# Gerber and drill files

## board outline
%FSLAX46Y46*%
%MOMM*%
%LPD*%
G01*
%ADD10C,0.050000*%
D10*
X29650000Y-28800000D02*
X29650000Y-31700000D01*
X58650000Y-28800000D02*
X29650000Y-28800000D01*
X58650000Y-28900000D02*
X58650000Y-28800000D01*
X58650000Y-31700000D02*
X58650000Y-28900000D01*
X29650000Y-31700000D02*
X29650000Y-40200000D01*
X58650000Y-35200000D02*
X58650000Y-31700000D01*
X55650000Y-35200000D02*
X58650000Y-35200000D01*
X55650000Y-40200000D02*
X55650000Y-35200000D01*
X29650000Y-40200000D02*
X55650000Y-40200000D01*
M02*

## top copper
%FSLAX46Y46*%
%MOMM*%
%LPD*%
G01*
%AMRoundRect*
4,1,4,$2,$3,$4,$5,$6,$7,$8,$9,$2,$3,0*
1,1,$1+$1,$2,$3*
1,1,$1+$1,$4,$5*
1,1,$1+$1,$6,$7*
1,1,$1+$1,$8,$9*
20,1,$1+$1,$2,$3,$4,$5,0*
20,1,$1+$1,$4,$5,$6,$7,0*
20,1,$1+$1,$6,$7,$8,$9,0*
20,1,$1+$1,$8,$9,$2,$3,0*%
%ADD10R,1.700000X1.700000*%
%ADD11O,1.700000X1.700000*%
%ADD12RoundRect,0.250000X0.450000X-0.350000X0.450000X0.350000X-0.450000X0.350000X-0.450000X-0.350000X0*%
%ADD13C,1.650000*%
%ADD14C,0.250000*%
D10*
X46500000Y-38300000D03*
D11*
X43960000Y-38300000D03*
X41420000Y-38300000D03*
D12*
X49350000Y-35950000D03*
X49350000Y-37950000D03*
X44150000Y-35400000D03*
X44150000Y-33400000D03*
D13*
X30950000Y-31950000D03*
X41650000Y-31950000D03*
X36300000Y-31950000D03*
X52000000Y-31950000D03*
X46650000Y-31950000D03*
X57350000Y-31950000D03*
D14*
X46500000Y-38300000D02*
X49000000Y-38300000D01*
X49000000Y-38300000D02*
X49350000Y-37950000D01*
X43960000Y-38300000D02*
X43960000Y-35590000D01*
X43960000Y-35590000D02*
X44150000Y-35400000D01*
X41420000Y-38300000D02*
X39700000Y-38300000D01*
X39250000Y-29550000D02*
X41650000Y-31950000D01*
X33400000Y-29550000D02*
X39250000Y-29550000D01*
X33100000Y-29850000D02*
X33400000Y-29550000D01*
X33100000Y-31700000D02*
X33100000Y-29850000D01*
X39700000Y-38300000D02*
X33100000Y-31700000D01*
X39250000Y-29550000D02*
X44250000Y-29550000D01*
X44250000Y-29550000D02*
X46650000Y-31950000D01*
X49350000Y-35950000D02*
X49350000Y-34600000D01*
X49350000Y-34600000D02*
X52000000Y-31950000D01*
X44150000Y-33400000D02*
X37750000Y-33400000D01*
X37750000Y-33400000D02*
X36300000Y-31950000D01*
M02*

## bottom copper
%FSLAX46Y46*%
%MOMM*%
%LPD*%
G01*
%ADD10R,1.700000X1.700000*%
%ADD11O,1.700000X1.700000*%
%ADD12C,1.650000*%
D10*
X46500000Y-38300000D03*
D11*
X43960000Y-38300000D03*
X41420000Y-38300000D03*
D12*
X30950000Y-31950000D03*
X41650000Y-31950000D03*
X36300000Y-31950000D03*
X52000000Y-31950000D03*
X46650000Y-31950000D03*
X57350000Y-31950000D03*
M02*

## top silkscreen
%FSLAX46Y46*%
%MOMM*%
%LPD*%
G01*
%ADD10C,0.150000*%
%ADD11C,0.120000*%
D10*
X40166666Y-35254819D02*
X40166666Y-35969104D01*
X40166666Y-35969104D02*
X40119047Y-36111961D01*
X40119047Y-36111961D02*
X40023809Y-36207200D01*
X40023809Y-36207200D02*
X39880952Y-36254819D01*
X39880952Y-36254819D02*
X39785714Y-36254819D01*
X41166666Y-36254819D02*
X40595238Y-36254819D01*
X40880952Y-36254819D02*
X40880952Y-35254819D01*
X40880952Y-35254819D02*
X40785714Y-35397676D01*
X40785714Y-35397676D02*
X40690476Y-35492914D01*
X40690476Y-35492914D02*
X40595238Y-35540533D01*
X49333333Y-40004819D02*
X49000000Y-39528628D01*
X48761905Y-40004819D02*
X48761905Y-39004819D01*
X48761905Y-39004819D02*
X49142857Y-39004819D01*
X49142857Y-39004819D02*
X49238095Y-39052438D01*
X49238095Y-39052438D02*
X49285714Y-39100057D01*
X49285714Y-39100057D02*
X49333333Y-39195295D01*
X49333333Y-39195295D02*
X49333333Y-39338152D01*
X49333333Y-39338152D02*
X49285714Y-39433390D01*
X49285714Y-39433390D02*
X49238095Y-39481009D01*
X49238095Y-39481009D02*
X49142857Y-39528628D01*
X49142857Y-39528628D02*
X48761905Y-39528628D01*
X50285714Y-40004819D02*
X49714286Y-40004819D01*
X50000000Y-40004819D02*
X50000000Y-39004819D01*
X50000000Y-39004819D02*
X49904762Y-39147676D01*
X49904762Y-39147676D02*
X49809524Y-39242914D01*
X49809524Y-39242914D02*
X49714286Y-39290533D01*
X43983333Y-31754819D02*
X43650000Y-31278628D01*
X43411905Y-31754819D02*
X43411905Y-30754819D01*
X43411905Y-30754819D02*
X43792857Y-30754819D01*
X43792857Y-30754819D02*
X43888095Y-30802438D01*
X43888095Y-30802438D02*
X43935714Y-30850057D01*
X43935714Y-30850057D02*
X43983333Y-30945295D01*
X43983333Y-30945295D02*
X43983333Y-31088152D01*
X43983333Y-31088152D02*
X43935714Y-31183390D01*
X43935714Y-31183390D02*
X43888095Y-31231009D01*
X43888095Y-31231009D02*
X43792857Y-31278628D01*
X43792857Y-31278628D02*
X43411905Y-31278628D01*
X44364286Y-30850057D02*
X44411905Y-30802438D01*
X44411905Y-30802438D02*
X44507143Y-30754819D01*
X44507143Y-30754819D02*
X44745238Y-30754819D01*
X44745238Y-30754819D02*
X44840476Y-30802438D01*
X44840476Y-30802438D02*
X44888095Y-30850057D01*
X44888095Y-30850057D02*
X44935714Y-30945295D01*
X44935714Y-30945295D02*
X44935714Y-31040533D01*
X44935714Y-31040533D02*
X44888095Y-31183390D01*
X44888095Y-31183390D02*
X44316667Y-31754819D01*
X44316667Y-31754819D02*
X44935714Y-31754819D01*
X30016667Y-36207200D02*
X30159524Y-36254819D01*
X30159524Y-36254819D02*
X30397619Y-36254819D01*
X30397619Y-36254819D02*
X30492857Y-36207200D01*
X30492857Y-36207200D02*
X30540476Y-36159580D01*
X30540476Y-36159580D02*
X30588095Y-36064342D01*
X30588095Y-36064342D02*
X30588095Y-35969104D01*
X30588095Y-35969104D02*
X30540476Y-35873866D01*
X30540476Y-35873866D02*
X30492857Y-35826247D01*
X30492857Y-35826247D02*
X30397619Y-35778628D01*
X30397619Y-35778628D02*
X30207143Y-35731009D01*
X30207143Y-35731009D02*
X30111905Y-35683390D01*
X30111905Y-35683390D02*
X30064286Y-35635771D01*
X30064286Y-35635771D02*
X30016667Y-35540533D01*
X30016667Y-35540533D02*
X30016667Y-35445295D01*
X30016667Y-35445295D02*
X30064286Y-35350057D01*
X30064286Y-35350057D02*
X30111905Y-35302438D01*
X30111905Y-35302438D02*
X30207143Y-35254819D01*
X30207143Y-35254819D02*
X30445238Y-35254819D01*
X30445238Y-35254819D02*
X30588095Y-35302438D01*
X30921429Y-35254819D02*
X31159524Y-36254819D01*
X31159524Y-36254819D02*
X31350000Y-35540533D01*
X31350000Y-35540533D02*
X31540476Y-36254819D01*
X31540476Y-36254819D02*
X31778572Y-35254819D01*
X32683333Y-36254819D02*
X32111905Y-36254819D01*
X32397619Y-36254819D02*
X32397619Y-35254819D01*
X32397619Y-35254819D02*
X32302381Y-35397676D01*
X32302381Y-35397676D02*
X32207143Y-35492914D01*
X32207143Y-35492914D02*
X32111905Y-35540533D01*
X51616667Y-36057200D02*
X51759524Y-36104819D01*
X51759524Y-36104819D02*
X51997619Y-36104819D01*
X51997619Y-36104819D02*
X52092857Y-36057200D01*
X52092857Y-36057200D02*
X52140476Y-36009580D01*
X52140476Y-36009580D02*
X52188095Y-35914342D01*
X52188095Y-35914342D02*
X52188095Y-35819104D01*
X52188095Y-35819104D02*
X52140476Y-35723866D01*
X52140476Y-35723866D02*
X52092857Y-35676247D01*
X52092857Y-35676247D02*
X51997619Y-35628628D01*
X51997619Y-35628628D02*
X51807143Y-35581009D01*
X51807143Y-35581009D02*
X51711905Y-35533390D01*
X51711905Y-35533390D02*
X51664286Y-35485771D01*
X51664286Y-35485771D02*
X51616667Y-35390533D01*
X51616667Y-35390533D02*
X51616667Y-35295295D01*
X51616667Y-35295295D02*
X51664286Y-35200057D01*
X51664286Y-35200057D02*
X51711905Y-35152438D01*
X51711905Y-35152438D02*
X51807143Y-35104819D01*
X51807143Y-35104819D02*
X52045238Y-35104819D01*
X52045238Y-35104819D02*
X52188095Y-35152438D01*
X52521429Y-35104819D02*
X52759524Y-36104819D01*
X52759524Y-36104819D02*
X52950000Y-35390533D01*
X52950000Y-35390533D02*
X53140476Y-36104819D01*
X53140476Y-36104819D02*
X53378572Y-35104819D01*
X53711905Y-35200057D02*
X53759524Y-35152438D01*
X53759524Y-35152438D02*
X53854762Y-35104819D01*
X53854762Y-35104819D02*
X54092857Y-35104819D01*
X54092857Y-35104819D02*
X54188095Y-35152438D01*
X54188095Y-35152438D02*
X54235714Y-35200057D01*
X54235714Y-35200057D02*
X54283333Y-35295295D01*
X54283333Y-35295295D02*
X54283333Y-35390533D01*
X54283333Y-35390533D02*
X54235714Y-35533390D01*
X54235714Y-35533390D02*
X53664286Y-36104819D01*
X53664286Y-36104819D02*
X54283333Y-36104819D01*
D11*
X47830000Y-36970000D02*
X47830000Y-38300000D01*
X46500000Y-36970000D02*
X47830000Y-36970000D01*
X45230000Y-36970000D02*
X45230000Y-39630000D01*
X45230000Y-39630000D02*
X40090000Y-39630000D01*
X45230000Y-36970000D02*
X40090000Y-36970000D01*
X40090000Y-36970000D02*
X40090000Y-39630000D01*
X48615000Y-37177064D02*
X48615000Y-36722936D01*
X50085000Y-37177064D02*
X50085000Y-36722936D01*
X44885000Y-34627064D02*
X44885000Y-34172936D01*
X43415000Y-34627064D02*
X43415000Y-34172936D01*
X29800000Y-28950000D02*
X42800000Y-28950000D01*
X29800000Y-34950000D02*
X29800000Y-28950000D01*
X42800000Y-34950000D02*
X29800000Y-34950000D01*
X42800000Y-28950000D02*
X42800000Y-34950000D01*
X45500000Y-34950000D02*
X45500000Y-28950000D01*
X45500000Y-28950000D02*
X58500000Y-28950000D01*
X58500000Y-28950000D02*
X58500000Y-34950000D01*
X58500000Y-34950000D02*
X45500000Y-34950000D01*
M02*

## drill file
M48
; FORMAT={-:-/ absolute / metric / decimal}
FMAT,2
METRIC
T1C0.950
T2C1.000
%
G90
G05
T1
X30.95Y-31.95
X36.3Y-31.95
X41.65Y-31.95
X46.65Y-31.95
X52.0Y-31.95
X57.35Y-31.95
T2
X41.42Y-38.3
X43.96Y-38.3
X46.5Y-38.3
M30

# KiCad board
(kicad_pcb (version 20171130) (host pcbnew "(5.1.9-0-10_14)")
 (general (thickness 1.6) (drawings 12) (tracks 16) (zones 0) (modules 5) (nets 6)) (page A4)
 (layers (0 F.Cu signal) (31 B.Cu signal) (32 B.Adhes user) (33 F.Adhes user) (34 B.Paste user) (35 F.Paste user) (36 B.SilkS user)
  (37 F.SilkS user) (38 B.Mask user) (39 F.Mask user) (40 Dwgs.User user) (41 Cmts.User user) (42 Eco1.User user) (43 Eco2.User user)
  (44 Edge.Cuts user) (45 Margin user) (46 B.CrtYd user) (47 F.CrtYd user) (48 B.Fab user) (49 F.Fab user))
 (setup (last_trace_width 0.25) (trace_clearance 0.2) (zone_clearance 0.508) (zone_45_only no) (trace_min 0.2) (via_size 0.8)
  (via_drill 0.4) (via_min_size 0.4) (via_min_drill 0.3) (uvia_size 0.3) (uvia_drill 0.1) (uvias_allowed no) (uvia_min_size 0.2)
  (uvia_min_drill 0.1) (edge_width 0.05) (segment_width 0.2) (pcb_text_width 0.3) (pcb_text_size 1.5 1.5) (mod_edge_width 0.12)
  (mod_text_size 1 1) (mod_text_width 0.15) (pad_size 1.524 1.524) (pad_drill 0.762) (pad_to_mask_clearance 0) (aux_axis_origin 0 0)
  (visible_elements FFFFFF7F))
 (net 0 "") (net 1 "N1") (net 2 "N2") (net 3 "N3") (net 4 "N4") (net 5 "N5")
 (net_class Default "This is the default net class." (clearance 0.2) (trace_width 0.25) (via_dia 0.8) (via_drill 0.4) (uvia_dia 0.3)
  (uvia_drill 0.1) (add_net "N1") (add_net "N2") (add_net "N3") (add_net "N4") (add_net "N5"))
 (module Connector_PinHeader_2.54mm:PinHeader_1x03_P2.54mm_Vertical (layer F.Cu) (at 46.5 38.3 270)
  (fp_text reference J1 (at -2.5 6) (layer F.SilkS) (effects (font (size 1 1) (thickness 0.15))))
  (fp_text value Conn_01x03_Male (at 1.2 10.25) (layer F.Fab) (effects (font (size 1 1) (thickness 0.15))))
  (fp_line (start -1.33 -1.33) (end 0 -1.33) (layer F.SilkS) (width 0.12))
  (fp_line (start -1.33 0) (end -1.33 -1.33) (layer F.SilkS) (width 0.12))
  (fp_line (start -1.33 1.27) (end 1.33 1.27) (layer F.SilkS) (width 0.12))
  (fp_line (start 1.33 1.27) (end 1.33 6.41) (layer F.SilkS) (width 0.12))
  (fp_line (start -1.33 1.27) (end -1.33 6.41) (layer F.SilkS) (width 0.12))
  (fp_line (start -1.33 6.41) (end 1.33 6.41) (layer F.SilkS) (width 0.12))
  (pad 1 thru_hole rect (at 0 0 270) (size 1.7 1.7) (drill 1) (layers *.Cu *.Mask) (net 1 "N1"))
  (pad 2 thru_hole oval (at 0 2.54 270) (size 1.7 1.7) (drill 1) (layers *.Cu *.Mask) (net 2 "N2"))
  (pad 3 thru_hole oval (at 0 5.08 270) (size 1.7 1.7) (drill 1) (layers *.Cu *.Mask) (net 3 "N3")))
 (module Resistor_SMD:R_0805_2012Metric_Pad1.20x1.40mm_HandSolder (layer F.Cu) (at 49.35 36.95 90)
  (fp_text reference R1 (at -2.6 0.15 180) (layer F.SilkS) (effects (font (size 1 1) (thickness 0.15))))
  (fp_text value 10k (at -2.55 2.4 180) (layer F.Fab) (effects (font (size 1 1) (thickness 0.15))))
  (fp_line (start -0.227064 -0.735) (end 0.227064 -0.735) (layer F.SilkS) (width 0.12))
  (fp_line (start -0.227064 0.735) (end 0.227064 0.735) (layer F.SilkS) (width 0.12))
  (pad 2 smd roundrect (at 1 0 90) (size 1.2 1.4) (layers F.Cu F.Paste F.Mask) (roundrect_rratio 0.208333) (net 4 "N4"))
  (pad 1 smd roundrect (at -1 0 90) (size 1.2 1.4) (layers F.Cu F.Paste F.Mask) (roundrect_rratio 0.208333) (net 1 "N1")))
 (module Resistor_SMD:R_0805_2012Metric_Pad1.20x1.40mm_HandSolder (layer F.Cu) (at 44.15 34.4 90)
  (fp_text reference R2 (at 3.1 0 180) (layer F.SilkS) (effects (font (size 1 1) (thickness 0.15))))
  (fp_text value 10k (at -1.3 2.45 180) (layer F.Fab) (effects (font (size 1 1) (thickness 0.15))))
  (fp_line (start -0.227064 0.735) (end 0.227064 0.735) (layer F.SilkS) (width 0.12))
  (fp_line (start -0.227064 -0.735) (end 0.227064 -0.735) (layer F.SilkS) (width 0.12))
  (pad 1 smd roundrect (at -1 0 90) (size 1.2 1.4) (layers F.Cu F.Paste F.Mask) (roundrect_rratio 0.208333) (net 2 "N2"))
  (pad 2 smd roundrect (at 1 0 90) (size 1.2 1.4) (layers F.Cu F.Paste F.Mask) (roundrect_rratio 0.208333) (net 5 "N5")))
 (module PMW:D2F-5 (layer F.Cu) (at 36.3 31.95 270)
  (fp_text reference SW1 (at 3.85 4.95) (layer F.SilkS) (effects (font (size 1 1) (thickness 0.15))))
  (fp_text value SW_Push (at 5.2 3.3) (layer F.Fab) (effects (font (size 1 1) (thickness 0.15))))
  (fp_line (start -3 6.5) (end -3 -6.5) (layer F.SilkS) (width 0.12))
  (fp_line (start 3 6.5) (end -3 6.5) (layer F.SilkS) (width 0.12))
  (fp_line (start 3 -6.5) (end 3 6.5) (layer F.SilkS) (width 0.12))
  (fp_line (start -3 -6.5) (end 3 -6.5) (layer F.SilkS) (width 0.12))
  (pad 3 thru_hole circle (at 0 5.35 270) (size 1.65 1.65) (drill 0.95) (layers *.Cu *.Mask))
  (pad 1 thru_hole circle (at 0 -5.35 270) (size 1.65 1.65) (drill 0.95) (layers *.Cu *.Mask) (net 3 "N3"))
  (pad 2 thru_hole circle (at 0 0 270) (size 1.65 1.65) (drill 0.95) (layers *.Cu *.Mask) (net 5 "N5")))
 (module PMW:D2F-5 (layer F.Cu) (at 52 31.95 90)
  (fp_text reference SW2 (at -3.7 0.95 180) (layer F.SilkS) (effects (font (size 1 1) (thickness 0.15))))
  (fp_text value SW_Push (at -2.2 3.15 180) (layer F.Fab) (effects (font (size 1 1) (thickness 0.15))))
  (fp_line (start -3 -6.5) (end 3 -6.5) (layer F.SilkS) (width 0.12))
  (fp_line (start 3 -6.5) (end 3 6.5) (layer F.SilkS) (width 0.12))
  (fp_line (start 3 6.5) (end -3 6.5) (layer F.SilkS) (width 0.12))
  (fp_line (start -3 6.5) (end -3 -6.5) (layer F.SilkS) (width 0.12))
  (pad 2 thru_hole circle (at 0 0 90) (size 1.65 1.65) (drill 0.95) (layers *.Cu *.Mask) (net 4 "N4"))
  (pad 1 thru_hole circle (at 0 -5.35 90) (size 1.65 1.65) (drill 0.95) (layers *.Cu *.Mask) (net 3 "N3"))
  (pad 3 thru_hole circle (at 0 5.35 90) (size 1.65 1.65) (drill 0.95) (layers *.Cu *.Mask)))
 (gr_line (start 29.65 28.8) (end 29.65 31.7) (angle 90) (layer Edge.Cuts) (width 0.05))
 (gr_line (start 58.65 28.8) (end 29.65 28.8) (angle 90) (layer Edge.Cuts) (width 0.05))
 (gr_line (start 58.65 28.9) (end 58.65 28.8) (angle 90) (layer Edge.Cuts) (width 0.05))
 (gr_line (start 58.65 31.7) (end 58.65 28.9) (angle 90) (layer Edge.Cuts) (width 0.05))
 (gr_line (start 29.65 31.7) (end 29.65 40.2) (angle 90) (layer Edge.Cuts) (width 0.05))
 (gr_line (start 58.65 35.2) (end 58.65 31.7) (angle 90) (layer Edge.Cuts) (width 0.05))
 (gr_line (start 55.65 35.2) (end 58.65 35.2) (angle 90) (layer Edge.Cuts) (width 0.05))
 (gr_line (start 55.65 40.2) (end 55.65 35.2) (angle 90) (layer Edge.Cuts) (width 0.05))
 (gr_line (start 29.65 40.2) (end 55.65 40.2) (angle 90) (layer Edge.Cuts) (width 0.05))
 (segment (start 46.5 38.3) (end 49 38.3) (width 0.25) (layer F.Cu) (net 1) (status C00000))
 (segment (start 49 38.3) (end 49.35 37.95) (width 0.25) (layer F.Cu) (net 1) (status C00000))
 (segment (start 43.96 38.3) (end 43.96 35.59) (width 0.25) (layer F.Cu) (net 2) (status C00000))
 (segment (start 43.96 35.59) (end 44.15 35.4) (width 0.25) (layer F.Cu) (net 2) (status C00000))
 (segment (start 41.42 38.3) (end 39.7 38.3) (width 0.25) (layer F.Cu) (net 3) (status 400000))
 (segment (start 39.25 29.55) (end 41.65 31.95) (width 0.25) (layer F.Cu) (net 3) (status 800000))
 (segment (start 33.4 29.55) (end 39.25 29.55) (width 0.25) (layer F.Cu) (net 3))
 (segment (start 33.1 29.85) (end 33.4 29.55) (width 0.25) (layer F.Cu) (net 3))
 (segment (start 33.1 31.7) (end 33.1 29.85) (width 0.25) (layer F.Cu) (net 3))
 (segment (start 39.7 38.3) (end 33.1 31.7) (width 0.25) (layer F.Cu) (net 3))
 (segment (start 39.25 29.55) (end 44.25 29.55) (width 0.25) (layer F.Cu) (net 3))
 (segment (start 44.25 29.55) (end 46.65 31.95) (width 0.25) (layer F.Cu) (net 3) (status 800000))
 (segment (start 49.35 35.95) (end 49.35 34.6) (width 0.25) (layer F.Cu) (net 4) (status 400000))
 (segment (start 49.35 34.6) (end 52 31.95) (width 0.25) (layer F.Cu) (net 4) (status 800000))
 (segment (start 44.15 33.4) (end 37.75 33.4) (width 0.25) (layer F.Cu) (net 5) (status 400000))
 (segment (start 37.75 33.4) (end 36.3 31.95) (width 0.25) (layer F.Cu) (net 5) (status 800000)))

